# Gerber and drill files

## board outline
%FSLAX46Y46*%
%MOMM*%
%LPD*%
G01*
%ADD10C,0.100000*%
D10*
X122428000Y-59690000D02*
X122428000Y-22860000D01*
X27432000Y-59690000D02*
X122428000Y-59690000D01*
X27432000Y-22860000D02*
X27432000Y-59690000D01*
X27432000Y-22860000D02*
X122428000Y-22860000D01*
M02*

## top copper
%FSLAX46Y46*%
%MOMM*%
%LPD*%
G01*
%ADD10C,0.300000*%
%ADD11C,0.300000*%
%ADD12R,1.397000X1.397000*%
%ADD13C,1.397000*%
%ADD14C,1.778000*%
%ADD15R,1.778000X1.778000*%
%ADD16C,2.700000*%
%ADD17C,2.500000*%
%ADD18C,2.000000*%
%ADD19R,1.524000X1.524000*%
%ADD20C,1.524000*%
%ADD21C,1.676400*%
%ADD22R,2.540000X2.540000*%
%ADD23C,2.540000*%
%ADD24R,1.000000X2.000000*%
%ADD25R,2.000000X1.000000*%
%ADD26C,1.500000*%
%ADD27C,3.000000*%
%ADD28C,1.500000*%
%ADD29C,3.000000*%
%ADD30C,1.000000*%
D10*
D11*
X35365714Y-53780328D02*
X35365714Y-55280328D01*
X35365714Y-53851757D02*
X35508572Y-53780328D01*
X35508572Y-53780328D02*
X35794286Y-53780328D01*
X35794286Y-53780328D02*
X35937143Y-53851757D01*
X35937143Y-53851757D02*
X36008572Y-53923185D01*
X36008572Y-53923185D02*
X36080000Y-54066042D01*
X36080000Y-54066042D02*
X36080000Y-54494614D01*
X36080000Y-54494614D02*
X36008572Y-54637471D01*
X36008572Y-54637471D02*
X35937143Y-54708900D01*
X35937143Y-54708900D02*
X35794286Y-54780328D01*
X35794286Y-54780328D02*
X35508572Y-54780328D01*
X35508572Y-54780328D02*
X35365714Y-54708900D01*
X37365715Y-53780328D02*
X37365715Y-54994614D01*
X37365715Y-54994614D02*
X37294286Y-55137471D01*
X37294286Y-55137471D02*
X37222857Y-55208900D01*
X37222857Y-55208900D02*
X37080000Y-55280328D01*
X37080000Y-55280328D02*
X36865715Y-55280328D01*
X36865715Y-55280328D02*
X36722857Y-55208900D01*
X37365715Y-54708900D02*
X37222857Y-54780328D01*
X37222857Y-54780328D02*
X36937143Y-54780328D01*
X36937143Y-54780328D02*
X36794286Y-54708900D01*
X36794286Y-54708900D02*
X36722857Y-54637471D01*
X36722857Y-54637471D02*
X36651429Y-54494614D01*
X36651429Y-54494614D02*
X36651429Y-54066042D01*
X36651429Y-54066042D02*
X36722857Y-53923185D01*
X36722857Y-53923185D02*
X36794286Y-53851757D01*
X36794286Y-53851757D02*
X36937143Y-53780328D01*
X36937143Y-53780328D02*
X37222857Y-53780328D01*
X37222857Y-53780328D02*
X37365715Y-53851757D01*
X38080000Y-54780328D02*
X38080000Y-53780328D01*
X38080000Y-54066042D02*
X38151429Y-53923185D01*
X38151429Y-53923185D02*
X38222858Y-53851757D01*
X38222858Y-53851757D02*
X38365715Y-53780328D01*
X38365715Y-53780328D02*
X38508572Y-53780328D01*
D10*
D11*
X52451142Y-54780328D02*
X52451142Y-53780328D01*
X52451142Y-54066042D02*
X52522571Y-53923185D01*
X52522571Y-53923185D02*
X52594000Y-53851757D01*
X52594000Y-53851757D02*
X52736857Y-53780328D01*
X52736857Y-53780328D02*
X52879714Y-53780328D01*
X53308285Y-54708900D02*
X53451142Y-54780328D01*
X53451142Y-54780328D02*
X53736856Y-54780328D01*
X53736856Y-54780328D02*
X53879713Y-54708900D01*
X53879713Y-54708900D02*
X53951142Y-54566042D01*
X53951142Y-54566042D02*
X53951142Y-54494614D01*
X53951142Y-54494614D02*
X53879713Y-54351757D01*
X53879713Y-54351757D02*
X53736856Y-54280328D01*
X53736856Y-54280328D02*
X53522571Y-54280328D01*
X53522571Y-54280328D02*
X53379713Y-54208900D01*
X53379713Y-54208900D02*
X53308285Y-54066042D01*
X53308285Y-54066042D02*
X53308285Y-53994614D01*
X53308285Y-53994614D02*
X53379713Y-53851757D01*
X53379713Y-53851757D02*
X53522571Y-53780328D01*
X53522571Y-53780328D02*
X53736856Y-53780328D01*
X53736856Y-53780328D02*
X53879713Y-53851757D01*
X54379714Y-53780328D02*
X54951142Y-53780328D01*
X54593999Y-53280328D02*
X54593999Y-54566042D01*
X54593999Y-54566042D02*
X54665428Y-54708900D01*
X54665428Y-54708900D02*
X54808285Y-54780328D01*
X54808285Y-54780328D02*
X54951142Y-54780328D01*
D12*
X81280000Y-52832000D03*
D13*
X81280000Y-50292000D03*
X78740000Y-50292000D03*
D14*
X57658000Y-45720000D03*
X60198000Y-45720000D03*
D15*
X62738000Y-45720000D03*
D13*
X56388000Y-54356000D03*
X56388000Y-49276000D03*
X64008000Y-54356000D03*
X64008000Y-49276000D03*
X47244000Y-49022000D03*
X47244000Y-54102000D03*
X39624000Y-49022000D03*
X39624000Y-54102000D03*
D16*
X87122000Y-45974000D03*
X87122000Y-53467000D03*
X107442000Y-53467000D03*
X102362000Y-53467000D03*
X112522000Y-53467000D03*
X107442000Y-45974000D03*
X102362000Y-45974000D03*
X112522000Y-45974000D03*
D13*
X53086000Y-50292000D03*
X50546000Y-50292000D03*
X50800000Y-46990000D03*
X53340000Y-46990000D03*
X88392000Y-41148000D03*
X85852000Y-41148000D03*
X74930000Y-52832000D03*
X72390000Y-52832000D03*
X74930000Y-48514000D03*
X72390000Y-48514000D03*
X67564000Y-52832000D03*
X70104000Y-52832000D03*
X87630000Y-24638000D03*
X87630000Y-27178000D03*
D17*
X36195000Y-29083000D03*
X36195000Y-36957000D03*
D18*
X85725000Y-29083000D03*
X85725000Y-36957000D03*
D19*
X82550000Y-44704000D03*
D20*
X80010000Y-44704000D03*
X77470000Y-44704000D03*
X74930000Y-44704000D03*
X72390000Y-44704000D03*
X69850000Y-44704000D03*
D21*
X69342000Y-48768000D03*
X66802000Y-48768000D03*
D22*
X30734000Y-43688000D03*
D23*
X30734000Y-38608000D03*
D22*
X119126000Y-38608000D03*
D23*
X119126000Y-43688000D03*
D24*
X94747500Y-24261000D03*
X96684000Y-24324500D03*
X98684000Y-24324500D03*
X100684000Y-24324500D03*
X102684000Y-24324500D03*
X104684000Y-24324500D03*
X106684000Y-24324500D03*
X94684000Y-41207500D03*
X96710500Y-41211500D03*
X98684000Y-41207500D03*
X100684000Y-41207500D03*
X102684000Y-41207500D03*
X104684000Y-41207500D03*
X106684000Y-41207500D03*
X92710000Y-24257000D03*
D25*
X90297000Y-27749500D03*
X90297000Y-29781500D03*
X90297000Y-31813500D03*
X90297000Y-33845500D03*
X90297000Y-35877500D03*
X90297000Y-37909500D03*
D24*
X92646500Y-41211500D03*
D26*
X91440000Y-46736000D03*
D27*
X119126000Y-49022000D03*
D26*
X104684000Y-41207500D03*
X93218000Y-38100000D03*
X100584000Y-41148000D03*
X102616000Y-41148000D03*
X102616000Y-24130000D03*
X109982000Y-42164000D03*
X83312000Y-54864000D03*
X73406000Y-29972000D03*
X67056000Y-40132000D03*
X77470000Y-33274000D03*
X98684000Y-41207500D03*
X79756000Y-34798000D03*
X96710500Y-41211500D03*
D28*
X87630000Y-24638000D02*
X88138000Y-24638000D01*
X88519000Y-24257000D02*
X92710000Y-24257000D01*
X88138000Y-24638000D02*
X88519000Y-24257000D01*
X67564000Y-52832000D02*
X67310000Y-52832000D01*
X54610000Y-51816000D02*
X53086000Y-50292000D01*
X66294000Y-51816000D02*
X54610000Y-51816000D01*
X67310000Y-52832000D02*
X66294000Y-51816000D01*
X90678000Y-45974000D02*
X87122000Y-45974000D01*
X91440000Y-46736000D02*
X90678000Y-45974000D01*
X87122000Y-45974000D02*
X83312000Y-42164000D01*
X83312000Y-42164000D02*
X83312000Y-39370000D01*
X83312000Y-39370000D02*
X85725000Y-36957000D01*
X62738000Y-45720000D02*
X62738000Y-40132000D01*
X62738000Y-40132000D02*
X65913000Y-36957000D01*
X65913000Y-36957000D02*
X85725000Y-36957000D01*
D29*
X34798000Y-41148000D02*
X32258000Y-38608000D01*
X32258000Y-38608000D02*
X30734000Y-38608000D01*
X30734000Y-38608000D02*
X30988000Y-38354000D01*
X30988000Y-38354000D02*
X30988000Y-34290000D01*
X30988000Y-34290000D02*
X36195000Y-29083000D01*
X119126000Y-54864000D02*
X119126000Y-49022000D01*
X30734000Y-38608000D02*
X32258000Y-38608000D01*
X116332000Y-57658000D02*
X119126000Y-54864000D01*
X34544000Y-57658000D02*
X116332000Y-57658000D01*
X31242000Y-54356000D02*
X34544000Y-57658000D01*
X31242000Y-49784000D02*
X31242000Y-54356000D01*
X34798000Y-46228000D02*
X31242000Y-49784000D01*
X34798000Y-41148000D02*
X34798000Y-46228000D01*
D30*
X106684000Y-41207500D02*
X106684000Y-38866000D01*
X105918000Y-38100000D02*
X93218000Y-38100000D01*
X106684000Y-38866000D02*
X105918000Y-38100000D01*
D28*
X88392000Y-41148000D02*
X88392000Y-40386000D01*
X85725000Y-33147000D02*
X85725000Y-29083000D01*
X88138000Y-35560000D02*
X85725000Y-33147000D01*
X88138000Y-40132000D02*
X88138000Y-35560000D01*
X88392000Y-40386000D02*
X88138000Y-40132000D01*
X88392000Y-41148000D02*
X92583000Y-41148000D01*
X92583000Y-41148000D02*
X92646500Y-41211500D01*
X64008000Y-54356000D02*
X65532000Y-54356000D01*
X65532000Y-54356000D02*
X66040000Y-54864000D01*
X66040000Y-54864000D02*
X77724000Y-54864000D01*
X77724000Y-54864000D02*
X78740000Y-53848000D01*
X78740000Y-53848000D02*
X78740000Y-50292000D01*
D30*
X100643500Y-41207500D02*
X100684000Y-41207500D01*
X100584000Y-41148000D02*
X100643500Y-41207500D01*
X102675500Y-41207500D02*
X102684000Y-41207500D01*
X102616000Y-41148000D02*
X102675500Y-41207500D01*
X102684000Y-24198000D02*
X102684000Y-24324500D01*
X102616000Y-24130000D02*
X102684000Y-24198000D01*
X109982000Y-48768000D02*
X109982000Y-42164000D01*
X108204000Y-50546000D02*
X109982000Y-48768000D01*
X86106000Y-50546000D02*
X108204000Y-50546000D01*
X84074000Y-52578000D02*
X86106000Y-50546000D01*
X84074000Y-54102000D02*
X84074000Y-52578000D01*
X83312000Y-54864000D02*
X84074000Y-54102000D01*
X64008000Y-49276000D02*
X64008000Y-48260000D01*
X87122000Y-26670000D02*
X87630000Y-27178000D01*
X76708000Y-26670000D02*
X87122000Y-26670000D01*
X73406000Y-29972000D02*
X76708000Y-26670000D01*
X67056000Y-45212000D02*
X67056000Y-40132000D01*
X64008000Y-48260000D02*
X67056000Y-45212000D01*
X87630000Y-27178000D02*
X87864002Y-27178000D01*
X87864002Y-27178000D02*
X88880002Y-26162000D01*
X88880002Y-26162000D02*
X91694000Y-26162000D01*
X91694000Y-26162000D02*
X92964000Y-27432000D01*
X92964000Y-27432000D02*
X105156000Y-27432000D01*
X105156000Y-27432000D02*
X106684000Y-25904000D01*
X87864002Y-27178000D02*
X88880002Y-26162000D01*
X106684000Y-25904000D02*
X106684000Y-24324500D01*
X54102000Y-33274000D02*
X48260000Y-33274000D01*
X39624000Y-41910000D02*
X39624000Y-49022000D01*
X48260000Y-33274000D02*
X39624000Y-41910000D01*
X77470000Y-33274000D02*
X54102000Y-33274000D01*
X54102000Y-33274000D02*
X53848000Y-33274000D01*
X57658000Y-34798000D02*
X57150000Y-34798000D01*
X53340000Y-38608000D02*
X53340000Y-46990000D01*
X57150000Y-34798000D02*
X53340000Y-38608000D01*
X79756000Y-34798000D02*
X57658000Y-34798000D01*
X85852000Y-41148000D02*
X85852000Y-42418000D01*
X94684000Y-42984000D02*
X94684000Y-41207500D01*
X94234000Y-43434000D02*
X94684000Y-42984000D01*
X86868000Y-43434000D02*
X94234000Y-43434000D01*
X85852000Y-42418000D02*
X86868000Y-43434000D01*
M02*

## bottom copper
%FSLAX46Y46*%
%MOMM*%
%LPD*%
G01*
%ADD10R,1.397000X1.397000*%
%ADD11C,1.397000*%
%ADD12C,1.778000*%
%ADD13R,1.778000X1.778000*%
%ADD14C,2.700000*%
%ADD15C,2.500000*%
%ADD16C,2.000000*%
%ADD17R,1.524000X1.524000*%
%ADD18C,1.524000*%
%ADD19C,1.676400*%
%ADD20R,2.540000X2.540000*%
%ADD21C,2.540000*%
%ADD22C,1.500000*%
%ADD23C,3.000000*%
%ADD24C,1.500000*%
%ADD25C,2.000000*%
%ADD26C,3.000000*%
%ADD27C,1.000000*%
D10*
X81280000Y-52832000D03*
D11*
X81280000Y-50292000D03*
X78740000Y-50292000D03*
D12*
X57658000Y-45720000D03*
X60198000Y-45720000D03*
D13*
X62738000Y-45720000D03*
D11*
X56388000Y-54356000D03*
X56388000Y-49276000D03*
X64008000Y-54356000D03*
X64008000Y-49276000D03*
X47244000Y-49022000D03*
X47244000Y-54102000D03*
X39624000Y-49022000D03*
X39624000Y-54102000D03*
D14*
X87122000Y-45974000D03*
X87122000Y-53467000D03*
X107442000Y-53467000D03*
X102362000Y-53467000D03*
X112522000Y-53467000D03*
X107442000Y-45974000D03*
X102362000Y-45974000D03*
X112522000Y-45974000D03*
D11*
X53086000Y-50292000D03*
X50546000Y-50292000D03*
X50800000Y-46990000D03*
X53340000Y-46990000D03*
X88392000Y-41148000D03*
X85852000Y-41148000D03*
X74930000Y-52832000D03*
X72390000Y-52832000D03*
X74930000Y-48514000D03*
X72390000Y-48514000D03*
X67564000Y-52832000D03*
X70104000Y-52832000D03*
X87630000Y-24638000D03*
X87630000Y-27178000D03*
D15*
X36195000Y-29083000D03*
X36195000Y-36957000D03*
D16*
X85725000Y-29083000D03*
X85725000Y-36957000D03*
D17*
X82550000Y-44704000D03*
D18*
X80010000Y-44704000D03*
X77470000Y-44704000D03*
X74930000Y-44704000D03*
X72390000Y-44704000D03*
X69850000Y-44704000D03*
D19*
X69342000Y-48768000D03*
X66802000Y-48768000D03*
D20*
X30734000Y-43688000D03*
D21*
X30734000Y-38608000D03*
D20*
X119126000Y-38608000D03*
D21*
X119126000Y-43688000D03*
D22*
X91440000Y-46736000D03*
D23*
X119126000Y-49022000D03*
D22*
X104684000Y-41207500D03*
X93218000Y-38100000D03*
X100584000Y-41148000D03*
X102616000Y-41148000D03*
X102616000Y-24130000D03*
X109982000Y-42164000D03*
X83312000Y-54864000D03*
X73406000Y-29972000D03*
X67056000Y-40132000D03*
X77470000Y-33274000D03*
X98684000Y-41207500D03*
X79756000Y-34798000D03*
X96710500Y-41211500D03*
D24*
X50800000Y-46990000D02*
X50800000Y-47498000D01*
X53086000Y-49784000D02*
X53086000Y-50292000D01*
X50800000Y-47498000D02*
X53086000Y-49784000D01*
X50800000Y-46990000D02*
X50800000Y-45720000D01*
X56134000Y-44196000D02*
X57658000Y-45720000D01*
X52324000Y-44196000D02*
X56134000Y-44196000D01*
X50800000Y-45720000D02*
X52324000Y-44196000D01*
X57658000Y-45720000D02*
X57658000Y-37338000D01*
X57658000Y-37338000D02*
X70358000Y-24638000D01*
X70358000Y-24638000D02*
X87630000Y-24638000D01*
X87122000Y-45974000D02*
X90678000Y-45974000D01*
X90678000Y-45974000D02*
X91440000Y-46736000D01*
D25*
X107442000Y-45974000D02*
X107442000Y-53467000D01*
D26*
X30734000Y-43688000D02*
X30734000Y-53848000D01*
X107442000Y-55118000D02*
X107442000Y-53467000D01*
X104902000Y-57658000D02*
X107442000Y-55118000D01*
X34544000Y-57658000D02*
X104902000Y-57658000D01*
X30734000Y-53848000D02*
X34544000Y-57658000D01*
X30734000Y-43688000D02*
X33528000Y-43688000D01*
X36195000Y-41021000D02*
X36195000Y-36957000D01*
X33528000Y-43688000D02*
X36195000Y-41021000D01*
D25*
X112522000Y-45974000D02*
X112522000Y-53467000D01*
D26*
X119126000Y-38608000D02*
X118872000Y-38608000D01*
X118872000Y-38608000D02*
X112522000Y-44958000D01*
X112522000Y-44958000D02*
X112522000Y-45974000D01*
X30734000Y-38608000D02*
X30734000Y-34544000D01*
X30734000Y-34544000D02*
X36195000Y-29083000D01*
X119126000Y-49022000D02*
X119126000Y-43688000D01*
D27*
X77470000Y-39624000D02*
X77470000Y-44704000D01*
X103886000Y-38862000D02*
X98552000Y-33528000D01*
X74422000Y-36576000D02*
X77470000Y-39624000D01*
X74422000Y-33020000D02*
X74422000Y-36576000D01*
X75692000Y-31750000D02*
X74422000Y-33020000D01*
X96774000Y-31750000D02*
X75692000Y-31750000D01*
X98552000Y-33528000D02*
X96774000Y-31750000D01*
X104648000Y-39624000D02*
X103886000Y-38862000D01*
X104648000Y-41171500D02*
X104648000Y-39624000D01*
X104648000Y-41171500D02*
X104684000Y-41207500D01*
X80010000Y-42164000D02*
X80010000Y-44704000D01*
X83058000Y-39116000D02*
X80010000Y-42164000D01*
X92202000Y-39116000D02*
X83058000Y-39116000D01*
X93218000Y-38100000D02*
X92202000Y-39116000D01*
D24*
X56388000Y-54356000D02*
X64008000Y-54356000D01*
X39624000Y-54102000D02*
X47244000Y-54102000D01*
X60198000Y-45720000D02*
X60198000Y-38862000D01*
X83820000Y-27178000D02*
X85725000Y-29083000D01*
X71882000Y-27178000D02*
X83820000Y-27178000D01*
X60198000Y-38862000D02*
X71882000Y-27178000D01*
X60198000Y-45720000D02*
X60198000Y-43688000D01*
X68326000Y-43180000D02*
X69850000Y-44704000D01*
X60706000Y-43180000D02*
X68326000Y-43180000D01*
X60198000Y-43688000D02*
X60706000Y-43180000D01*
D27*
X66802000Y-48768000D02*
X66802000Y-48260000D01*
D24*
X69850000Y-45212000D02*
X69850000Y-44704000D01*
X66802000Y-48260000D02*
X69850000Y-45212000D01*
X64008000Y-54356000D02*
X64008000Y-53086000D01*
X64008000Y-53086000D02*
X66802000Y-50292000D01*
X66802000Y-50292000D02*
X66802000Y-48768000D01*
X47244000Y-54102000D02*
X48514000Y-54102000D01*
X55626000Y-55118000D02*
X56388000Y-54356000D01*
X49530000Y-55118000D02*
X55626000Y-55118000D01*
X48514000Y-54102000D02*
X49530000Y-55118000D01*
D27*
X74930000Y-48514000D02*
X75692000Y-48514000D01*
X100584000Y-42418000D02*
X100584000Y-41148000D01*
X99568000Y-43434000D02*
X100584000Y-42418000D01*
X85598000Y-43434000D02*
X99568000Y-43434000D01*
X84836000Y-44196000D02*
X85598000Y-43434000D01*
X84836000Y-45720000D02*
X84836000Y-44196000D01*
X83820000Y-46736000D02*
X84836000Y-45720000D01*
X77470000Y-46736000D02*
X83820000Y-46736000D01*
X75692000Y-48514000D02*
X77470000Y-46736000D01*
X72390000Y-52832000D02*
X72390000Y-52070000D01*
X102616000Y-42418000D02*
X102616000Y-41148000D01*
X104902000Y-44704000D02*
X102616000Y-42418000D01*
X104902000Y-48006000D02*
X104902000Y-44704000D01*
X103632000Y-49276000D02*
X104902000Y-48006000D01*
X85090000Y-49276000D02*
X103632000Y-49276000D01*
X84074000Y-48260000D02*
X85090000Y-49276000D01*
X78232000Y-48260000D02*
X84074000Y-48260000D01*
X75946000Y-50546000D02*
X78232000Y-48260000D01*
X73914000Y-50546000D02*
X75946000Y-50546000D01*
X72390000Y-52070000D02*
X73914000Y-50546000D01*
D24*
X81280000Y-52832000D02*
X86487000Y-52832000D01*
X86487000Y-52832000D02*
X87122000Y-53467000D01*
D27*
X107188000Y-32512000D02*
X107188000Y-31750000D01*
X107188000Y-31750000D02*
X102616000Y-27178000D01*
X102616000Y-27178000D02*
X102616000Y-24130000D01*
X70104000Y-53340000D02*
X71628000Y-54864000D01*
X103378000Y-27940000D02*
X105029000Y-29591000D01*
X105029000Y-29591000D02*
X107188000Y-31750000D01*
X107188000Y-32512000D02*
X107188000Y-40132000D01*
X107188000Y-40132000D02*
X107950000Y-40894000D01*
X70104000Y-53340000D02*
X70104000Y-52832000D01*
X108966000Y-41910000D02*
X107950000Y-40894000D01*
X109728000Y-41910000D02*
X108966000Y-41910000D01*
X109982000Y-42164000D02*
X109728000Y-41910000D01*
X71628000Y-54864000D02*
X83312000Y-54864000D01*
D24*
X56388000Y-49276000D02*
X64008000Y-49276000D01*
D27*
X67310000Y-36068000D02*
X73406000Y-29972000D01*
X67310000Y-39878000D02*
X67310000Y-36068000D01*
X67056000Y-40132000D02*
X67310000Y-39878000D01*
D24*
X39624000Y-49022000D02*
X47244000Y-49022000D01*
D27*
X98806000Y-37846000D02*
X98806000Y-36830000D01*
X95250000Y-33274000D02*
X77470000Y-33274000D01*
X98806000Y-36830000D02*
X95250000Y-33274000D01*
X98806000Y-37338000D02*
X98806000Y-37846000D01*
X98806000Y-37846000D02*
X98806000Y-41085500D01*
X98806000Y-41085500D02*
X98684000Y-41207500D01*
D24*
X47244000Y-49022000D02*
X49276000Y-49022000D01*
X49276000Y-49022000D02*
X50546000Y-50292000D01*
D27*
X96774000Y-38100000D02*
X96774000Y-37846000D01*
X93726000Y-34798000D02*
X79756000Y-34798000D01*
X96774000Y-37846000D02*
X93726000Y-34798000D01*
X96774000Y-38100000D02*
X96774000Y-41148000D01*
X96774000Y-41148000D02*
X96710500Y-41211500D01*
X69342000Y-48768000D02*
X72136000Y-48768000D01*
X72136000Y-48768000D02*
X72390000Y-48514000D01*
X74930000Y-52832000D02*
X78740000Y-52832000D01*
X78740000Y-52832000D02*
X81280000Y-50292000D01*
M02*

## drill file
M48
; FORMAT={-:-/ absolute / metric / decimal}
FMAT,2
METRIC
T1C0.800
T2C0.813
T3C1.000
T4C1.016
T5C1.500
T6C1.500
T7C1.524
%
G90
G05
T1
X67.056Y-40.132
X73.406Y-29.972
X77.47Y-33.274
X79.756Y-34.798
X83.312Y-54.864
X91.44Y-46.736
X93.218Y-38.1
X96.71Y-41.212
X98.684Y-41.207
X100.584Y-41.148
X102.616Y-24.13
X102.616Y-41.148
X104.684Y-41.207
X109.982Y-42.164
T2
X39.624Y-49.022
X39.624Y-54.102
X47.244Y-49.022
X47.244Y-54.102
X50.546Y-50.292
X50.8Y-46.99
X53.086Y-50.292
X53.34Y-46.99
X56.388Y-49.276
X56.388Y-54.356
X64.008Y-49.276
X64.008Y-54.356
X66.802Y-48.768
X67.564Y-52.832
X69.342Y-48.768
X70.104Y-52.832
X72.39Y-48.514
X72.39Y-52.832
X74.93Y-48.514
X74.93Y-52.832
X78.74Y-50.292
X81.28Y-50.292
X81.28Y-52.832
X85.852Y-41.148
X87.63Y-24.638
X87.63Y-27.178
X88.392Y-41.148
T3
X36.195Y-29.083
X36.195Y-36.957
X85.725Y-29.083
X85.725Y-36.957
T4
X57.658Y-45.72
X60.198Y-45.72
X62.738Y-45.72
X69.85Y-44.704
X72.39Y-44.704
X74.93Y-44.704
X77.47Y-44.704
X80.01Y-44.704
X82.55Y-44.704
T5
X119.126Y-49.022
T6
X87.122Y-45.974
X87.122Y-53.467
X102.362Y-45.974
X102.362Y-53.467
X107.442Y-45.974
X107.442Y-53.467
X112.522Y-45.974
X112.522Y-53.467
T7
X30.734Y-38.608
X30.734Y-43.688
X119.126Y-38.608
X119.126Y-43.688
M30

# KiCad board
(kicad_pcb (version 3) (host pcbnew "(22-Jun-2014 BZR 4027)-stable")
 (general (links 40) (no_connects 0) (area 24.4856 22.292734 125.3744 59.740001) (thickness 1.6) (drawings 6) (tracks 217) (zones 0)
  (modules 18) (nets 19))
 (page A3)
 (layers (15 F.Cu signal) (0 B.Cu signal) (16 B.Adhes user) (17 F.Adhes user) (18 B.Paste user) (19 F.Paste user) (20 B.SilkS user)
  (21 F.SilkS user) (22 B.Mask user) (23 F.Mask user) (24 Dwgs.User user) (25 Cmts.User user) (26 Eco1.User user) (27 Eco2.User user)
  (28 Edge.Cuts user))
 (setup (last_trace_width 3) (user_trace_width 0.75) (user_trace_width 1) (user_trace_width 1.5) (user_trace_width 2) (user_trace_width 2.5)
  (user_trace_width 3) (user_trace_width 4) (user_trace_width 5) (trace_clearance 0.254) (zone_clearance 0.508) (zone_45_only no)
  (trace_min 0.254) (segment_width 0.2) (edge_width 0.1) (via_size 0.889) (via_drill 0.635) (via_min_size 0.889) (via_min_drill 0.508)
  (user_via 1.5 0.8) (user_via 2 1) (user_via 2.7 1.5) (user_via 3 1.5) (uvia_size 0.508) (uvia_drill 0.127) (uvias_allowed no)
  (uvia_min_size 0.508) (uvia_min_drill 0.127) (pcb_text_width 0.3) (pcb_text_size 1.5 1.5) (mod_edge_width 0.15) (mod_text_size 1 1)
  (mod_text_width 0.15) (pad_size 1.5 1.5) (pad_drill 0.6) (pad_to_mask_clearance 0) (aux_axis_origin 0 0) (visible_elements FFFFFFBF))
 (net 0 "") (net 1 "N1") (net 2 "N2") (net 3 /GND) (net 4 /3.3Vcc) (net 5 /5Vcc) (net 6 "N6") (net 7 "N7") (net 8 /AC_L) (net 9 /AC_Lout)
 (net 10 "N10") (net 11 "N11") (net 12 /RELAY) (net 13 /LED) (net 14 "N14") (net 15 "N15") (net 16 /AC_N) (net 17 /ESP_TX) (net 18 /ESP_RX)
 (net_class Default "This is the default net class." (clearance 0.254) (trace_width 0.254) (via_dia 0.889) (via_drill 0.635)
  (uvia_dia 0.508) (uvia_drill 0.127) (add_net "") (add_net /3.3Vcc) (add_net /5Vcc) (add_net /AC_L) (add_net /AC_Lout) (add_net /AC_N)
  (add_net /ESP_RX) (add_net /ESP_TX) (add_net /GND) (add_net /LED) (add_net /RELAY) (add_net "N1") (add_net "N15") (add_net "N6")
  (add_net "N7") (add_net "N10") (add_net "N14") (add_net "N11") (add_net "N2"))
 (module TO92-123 (layer F.Cu) (at 80.01 51.562 270)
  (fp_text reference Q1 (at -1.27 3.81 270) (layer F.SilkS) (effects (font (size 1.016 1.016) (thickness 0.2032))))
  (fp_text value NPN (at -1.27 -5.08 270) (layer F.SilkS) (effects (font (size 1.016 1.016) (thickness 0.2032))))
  (pad 3 thru_hole rect (at 1.27 -1.27 270) (size 1.397 1.397) (drill 0.8128) (layers *.Cu *.Mask F.SilkS) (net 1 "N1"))
  (pad 2 thru_hole circle (at -1.27 -1.27 270) (size 1.397 1.397) (drill 0.8128) (layers *.Cu *.Mask F.SilkS) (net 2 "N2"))
  (pad 1 thru_hole circle (at -1.27 1.27 270) (size 1.397 1.397) (drill 0.8128) (layers *.Cu *.Mask F.SilkS) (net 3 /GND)))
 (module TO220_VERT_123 (layer F.Cu) (at 60.198 45.72 90)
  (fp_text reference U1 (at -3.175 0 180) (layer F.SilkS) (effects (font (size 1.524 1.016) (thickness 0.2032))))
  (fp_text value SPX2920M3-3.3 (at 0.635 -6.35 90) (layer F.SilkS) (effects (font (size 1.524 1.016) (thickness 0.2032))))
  (pad 3 thru_hole circle (at 0 -2.54 90) (size 1.778 1.778) (drill 1.016) (layers *.Cu *.Mask F.SilkS) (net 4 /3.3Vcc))
  (pad 2 thru_hole circle (at 0 0 90) (size 1.778 1.778) (drill 1.016) (layers *.Cu *.Mask F.SilkS) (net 3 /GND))
  (pad 1 thru_hole rect (at 0 2.54 90) (size 1.778 1.778) (drill 1.016) (layers *.Cu *.Mask F.SilkS) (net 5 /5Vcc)))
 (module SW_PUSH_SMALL (layer F.Cu) (at 60.198 51.816 180)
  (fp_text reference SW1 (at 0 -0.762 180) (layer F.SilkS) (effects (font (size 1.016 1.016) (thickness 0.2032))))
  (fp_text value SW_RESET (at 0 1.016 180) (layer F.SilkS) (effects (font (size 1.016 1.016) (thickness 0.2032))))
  (pad 1 thru_hole circle (at 3.81 -2.54 180) (size 1.397 1.397) (drill 0.8128) (layers *.Cu *.Mask F.SilkS) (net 3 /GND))
  (pad 2 thru_hole circle (at 3.81 2.54 180) (size 1.397 1.397) (drill 0.8128) (layers *.Cu *.Mask F.SilkS) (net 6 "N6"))
  (pad 1 thru_hole circle (at -3.81 -2.54 180) (size 1.397 1.397) (drill 0.8128) (layers *.Cu *.Mask F.SilkS) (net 3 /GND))
  (pad 2 thru_hole circle (at -3.81 2.54 180) (size 1.397 1.397) (drill 0.8128) (layers *.Cu *.Mask F.SilkS) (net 6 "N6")))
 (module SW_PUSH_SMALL (layer F.Cu) (at 43.434 51.562)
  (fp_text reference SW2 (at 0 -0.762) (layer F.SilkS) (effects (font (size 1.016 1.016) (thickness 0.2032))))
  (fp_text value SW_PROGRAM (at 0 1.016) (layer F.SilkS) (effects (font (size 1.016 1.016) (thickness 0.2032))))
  (pad 1 thru_hole circle (at 3.81 -2.54) (size 1.397 1.397) (drill 0.8128) (layers *.Cu *.Mask F.SilkS) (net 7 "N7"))
  (pad 2 thru_hole circle (at 3.81 2.54) (size 1.397 1.397) (drill 0.8128) (layers *.Cu *.Mask F.SilkS) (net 3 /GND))
  (pad 1 thru_hole circle (at -3.81 -2.54) (size 1.397 1.397) (drill 0.8128) (layers *.Cu *.Mask F.SilkS) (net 7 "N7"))
  (pad 2 thru_hole circle (at -3.81 2.54) (size 1.397 1.397) (drill 0.8128) (layers *.Cu *.Mask F.SilkS) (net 3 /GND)))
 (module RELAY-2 (layer F.Cu) (at 88.646 44.196)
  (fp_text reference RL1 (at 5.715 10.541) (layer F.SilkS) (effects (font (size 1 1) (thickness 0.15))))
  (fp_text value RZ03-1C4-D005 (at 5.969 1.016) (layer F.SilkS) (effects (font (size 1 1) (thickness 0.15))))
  (pad 1 thru_hole circle (at -1.524 1.778) (size 2.7 2.7) (drill 1.5) (layers *.Cu *.Mask F.SilkS) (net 5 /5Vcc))
  (pad 2 thru_hole circle (at -1.524 9.271) (size 2.7 2.7) (drill 1.5) (layers *.Cu *.Mask F.SilkS) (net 1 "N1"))
  (pad 11 thru_hole circle (at 18.796 9.271) (size 2.7 2.7) (drill 1.5) (layers *.Cu *.Mask F.SilkS) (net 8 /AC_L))
  (pad 12 thru_hole circle (at 13.716 9.271) (size 2.7 2.7) (drill 1.5) (layers *.Cu *.Mask F.SilkS))
  (pad 14 thru_hole circle (at 23.876 9.271) (size 2.7 2.7) (drill 1.5) (layers *.Cu *.Mask F.SilkS) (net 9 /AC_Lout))
  (pad 11 thru_hole circle (at 18.796 1.778) (size 2.7 2.7) (drill 1.5) (layers *.Cu *.Mask F.SilkS) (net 8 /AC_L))
  (pad 12 thru_hole circle (at 13.716 1.778) (size 2.7 2.7) (drill 1.5) (layers *.Cu *.Mask F.SilkS))
  (pad 14 thru_hole circle (at 23.876 1.778) (size 2.7 2.7) (drill 1.5) (layers *.Cu *.Mask F.SilkS) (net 9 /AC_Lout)))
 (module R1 (layer F.Cu) (at 51.816 50.292 180) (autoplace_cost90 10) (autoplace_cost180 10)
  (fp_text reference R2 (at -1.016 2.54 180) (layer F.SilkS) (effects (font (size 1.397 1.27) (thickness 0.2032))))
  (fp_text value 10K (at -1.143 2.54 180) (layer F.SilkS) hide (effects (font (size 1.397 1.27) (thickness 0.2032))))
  (pad 1 thru_hole circle (at -1.27 0 180) (size 1.397 1.397) (drill 0.8128) (layers *.Cu *.Mask F.SilkS) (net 4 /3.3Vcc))
  (pad 2 thru_hole circle (at 1.27 0 180) (size 1.397 1.397) (drill 0.8128) (layers *.Cu *.Mask F.SilkS) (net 7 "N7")))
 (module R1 (layer F.Cu) (at 52.07 46.99) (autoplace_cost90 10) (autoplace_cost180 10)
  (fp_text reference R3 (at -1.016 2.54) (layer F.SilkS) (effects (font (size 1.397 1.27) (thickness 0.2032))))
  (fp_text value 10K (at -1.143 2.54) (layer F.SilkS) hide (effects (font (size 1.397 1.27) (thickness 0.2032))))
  (pad 1 thru_hole circle (at -1.27 0) (size 1.397 1.397) (drill 0.8128) (layers *.Cu *.Mask F.SilkS) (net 4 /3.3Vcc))
  (pad 2 thru_hole circle (at 1.27 0) (size 1.397 1.397) (drill 0.8128) (layers *.Cu *.Mask F.SilkS) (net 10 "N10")))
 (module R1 (layer F.Cu) (at 87.122 41.148 180) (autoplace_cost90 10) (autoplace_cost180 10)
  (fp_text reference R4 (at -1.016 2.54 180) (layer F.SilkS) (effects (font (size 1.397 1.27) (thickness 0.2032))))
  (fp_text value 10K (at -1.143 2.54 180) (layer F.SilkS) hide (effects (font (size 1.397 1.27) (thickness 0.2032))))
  (pad 1 thru_hole circle (at -1.27 0 180) (size 1.397 1.397) (drill 0.8128) (layers *.Cu *.Mask F.SilkS) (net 3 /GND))
  (pad 2 thru_hole circle (at 1.27 0 180) (size 1.397 1.397) (drill 0.8128) (layers *.Cu *.Mask F.SilkS) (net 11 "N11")))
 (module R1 (layer F.Cu) (at 73.66 52.832 180) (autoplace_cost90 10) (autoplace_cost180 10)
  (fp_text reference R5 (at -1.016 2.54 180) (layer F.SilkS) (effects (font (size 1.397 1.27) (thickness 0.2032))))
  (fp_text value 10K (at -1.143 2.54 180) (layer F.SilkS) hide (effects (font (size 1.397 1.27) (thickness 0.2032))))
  (pad 1 thru_hole circle (at -1.27 0 180) (size 1.397 1.397) (drill 0.8128) (layers *.Cu *.Mask F.SilkS) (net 2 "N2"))
  (pad 2 thru_hole circle (at 1.27 0 180) (size 1.397 1.397) (drill 0.8128) (layers *.Cu *.Mask F.SilkS) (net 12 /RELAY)))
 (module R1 (layer F.Cu) (at 73.66 48.514 180) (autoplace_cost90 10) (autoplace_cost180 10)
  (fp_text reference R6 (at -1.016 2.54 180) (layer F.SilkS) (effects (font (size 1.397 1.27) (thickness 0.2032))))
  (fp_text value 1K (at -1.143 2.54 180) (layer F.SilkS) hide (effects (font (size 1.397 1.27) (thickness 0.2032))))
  (pad 1 thru_hole circle (at -1.27 0 180) (size 1.397 1.397) (drill 0.8128) (layers *.Cu *.Mask F.SilkS) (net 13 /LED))
  (pad 2 thru_hole circle (at 1.27 0 180) (size 1.397 1.397) (drill 0.8128) (layers *.Cu *.Mask F.SilkS) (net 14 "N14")))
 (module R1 (layer F.Cu) (at 68.834 52.832) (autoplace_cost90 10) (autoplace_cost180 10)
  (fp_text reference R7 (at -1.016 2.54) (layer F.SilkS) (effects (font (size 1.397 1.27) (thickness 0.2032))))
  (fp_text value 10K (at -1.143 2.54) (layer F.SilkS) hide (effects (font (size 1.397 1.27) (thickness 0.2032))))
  (pad 1 thru_hole circle (at -1.27 0) (size 1.397 1.397) (drill 0.8128) (layers *.Cu *.Mask F.SilkS) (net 4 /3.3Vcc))
  (pad 2 thru_hole circle (at 1.27 0) (size 1.397 1.397) (drill 0.8128) (layers *.Cu *.Mask F.SilkS) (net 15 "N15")))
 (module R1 (layer F.Cu) (at 87.63 25.908 270) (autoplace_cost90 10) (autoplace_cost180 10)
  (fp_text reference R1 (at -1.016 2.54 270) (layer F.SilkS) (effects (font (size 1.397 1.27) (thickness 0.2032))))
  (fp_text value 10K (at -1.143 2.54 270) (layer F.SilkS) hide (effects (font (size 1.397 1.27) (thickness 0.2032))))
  (pad 1 thru_hole circle (at -1.27 0 270) (size 1.397 1.397) (drill 0.8128) (layers *.Cu *.Mask F.SilkS) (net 4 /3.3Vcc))
  (pad 2 thru_hole circle (at 1.27 0 270) (size 1.397 1.397) (drill 0.8128) (layers *.Cu *.Mask F.SilkS) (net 6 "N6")))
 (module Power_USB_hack (layer F.Cu) (at 60.96 33.02)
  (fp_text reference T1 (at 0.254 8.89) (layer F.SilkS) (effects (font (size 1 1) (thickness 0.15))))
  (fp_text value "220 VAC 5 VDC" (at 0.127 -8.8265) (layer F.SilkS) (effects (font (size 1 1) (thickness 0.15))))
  (pad 1 thru_hole circle (at -24.765 -3.937) (size 2.5 2.5) (drill 1) (layers *.Cu *.Mask F.SilkS) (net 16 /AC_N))
  (pad 2 thru_hole circle (at -24.765 3.937) (size 2.5 2.5) (drill 1) (layers *.Cu *.Mask F.SilkS) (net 8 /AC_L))
  (pad 4 thru_hole circle (at 24.765 -3.937) (size 2 2) (drill 1) (layers *.Cu *.Mask F.SilkS) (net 3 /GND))
  (pad 3 thru_hole circle (at 24.765 3.937) (size 2 2) (drill 1) (layers *.Cu *.Mask F.SilkS) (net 5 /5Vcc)))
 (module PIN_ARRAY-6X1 (layer F.Cu) (at 76.2 44.704 180)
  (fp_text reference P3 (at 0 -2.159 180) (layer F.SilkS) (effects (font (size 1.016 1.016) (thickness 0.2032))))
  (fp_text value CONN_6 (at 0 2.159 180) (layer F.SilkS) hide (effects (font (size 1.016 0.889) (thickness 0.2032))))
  (pad 1 thru_hole rect (at -6.35 0 180) (size 1.524 1.524) (drill 1.016) (layers *.Cu *.Mask F.SilkS))
  (pad 2 thru_hole circle (at -3.81 0 180) (size 1.524 1.524) (drill 1.016) (layers *.Cu *.Mask F.SilkS) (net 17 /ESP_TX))
  (pad 3 thru_hole circle (at -1.27 0 180) (size 1.524 1.524) (drill 1.016) (layers *.Cu *.Mask F.SilkS) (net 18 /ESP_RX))
  (pad 4 thru_hole circle (at 1.27 0 180) (size 1.524 1.524) (drill 1.016) (layers *.Cu *.Mask F.SilkS))
  (pad 5 thru_hole circle (at 3.81 0 180) (size 1.524 1.524) (drill 1.016) (layers *.Cu *.Mask F.SilkS))
  (pad 6 thru_hole circle (at 6.35 0 180) (size 1.524 1.524) (drill 1.016) (layers *.Cu *.Mask F.SilkS) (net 3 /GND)))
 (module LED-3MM (layer F.Cu) (at 68.072 48.768 180)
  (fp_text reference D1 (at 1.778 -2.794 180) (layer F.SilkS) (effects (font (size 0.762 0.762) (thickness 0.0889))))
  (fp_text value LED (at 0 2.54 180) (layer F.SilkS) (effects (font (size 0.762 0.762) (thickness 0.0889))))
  (pad 1 thru_hole circle (at -1.27 0 180) (size 1.6764 1.6764) (drill 0.8128) (layers *.Cu *.Mask F.SilkS) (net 14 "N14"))
  (pad 2 thru_hole circle (at 1.27 0 180) (size 1.6764 1.6764) (drill 0.8128) (layers *.Cu *.Mask F.SilkS) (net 3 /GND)))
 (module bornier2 (layer F.Cu) (at 30.734 41.148 90)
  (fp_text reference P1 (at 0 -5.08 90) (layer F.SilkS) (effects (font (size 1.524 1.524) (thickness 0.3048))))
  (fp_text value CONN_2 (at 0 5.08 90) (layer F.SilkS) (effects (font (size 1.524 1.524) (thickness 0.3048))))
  (pad 1 thru_hole rect (at -2.54 0 90) (size 2.54 2.54) (drill 1.524) (layers *.Cu *.Mask F.SilkS) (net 8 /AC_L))
  (pad 2 thru_hole circle (at 2.54 0 90) (size 2.54 2.54) (drill 1.524) (layers *.Cu *.Mask F.SilkS) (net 16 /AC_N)))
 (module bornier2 (layer F.Cu) (at 119.126 41.148 270)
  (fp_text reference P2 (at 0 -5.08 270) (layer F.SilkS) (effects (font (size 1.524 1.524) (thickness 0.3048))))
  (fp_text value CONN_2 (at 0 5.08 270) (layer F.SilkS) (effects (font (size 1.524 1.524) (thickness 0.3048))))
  (pad 1 thru_hole rect (at -2.54 0 270) (size 2.54 2.54) (drill 1.524) (layers *.Cu *.Mask F.SilkS) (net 9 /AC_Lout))
  (pad 2 thru_hole circle (at 2.54 0 270) (size 2.54 2.54) (drill 1.524) (layers *.Cu *.Mask F.SilkS) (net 16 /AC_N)))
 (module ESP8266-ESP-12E (layer F.Cu) (at 102.87 32.766 270)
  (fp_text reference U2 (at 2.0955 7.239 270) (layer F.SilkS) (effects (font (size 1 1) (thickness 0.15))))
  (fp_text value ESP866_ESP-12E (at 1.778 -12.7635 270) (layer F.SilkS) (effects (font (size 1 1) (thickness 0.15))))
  (pad 7 smd rect (at -8.505 8.1225 270) (size 2 1) (layers F.Cu F.Paste F.Mask))
  (pad 6 smd rect (at -8.4415 6.186 270) (size 2 1) (layers F.Cu F.Paste F.Mask))
  (pad 5 smd rect (at -8.4415 4.186 270) (size 2 1) (layers F.Cu F.Paste F.Mask))
  (pad 4 smd rect (at -8.4415 2.186 270) (size 2 1) (layers F.Cu F.Paste F.Mask))
  (pad 3 smd rect (at -8.4415 0.186 270) (size 2 1) (layers F.Cu F.Paste F.Mask) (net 15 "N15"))
  (pad 2 smd rect (at -8.4415 -1.814 270) (size 2 1) (layers F.Cu F.Paste F.Mask))
  (pad 1 smd rect (at -8.4415 -3.814 270) (size 2 1) (layers F.Cu F.Paste F.Mask) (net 6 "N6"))
  (pad 16 smd rect (at 8.4415 8.186 270) (size 2 1) (layers F.Cu F.Paste F.Mask) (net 11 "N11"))
  (pad 17 smd rect (at 8.4455 6.1595 270) (size 2 1) (layers F.Cu F.Paste F.Mask) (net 10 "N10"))
  (pad 18 smd rect (at 8.4415 4.186 270) (size 2 1) (layers F.Cu F.Paste F.Mask) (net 7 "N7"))
  (pad 19 smd rect (at 8.4415 2.186 270) (size 2 1) (layers F.Cu F.Paste F.Mask) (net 13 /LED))
  (pad 20 smd rect (at 8.4415 0.186 270) (size 2 1) (layers F.Cu F.Paste F.Mask) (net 12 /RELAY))
  (pad 21 smd rect (at 8.4415 -1.814 270) (size 2 1) (layers F.Cu F.Paste F.Mask) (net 18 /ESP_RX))
  (pad 22 smd rect (at 8.4415 -3.814 270) (size 2 1) (layers F.Cu F.Paste F.Mask) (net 17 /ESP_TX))
  (pad 8 smd rect (at -8.509 10.16 270) (size 2 1) (layers F.Cu F.Paste F.Mask) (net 4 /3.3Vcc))
  (pad 9 smd rect (at -5.0165 12.573) (size 2 1) (layers F.Cu F.Paste F.Mask))
  (pad 10 smd rect (at -2.9845 12.573) (size 2 1) (layers F.Cu F.Paste F.Mask))
  (pad 11 smd rect (at -0.9525 12.573) (size 2 1) (layers F.Cu F.Paste F.Mask))
  (pad 12 smd rect (at 1.0795 12.573) (size 2 1) (layers F.Cu F.Paste F.Mask))
  (pad 13 smd rect (at 3.1115 12.573) (size 2 1) (layers F.Cu F.Paste F.Mask))
  (pad 14 smd rect (at 5.1435 12.573) (size 2 1) (layers F.Cu F.Paste F.Mask))
  (pad 15 smd rect (at 8.4455 10.2235 270) (size 2 1) (layers F.Cu F.Paste F.Mask) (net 3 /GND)))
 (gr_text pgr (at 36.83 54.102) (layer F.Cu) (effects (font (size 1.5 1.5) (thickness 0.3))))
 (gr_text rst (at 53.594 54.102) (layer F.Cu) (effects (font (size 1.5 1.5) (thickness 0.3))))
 (gr_line (start 122.428 59.69) (end 122.428 22.86) (angle 90) (layer Edge.Cuts) (width 0.1))
 (gr_line (start 27.432 59.69) (end 122.428 59.69) (angle 90) (layer Edge.Cuts) (width 0.1))
 (gr_line (start 27.432 22.86) (end 27.432 59.69) (angle 90) (layer Edge.Cuts) (width 0.1))
 (gr_line (start 27.432 22.86) (end 122.428 22.86) (angle 90) (layer Edge.Cuts) (width 0.1))
 (segment (start 87.63 24.638) (end 88.138 24.638) (width 1.5) (layer F.Cu) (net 4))
 (segment (start 88.519 24.257) (end 92.71 24.257) (width 1.5) (layer F.Cu) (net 4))
 (segment (start 88.138 24.638) (end 88.519 24.257) (width 1.5) (layer F.Cu) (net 4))
 (segment (start 67.564 52.832) (end 67.31 52.832) (width 1.5) (layer F.Cu) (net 4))
 (segment (start 54.61 51.816) (end 53.086 50.292) (width 1.5) (layer F.Cu) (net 4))
 (segment (start 66.294 51.816) (end 54.61 51.816) (width 1.5) (layer F.Cu) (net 4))
 (segment (start 67.31 52.832) (end 66.294 51.816) (width 1.5) (layer F.Cu) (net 4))
 (segment (start 50.8 46.99) (end 50.8 47.498) (width 1.5) (layer B.Cu) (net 4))
 (segment (start 53.086 49.784) (end 53.086 50.292) (width 1.5) (layer B.Cu) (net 4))
 (segment (start 50.8 47.498) (end 53.086 49.784) (width 1.5) (layer B.Cu) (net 4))
 (segment (start 50.8 46.99) (end 50.8 45.72) (width 1.5) (layer B.Cu) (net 4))
 (segment (start 56.134 44.196) (end 57.658 45.72) (width 1.5) (layer B.Cu) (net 4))
 (segment (start 52.324 44.196) (end 56.134 44.196) (width 1.5) (layer B.Cu) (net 4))
 (segment (start 50.8 45.72) (end 52.324 44.196) (width 1.5) (layer B.Cu) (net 4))
 (segment (start 57.658 45.72) (end 57.658 37.338) (width 1.5) (layer B.Cu) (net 4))
 (segment (start 57.658 37.338) (end 70.358 24.638) (width 1.5) (layer B.Cu) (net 4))
 (segment (start 70.358 24.638) (end 87.63 24.638) (width 1.5) (layer B.Cu) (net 4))
 (segment (start 87.122 45.974) (end 90.678 45.974) (width 1.5) (layer B.Cu) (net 5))
 (segment (start 90.678 45.974) (end 87.122 45.974) (width 1.5) (layer F.Cu) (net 5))
 (segment (start 91.44 46.736) (end 90.678 45.974) (width 1.5) (layer F.Cu) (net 5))
 (via (at 91.44 46.736) (size 1.5) (drill 0.8) (layers F.Cu B.Cu) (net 5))
 (segment (start 90.678 45.974) (end 91.44 46.736) (width 1.5) (layer B.Cu) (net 5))
 (segment (start 87.122 45.974) (end 83.312 42.164) (width 1.5) (layer F.Cu) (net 5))
 (segment (start 83.312 42.164) (end 83.312 39.37) (width 1.5) (layer F.Cu) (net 5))
 (segment (start 83.312 39.37) (end 85.725 36.957) (width 1.5) (layer F.Cu) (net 5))
 (segment (start 62.738 45.72) (end 62.738 40.132) (width 1.5) (layer F.Cu) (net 5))
 (segment (start 62.738 40.132) (end 65.913 36.957) (width 1.5) (layer F.Cu) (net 5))
 (segment (start 65.913 36.957) (end 85.725 36.957) (width 1.5) (layer F.Cu) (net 5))
 (segment (start 107.442 45.974) (end 107.442 53.467) (width 2) (layer B.Cu) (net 8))
 (segment (start 30.734 43.688) (end 30.734 53.848) (width 3) (layer B.Cu) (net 8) (status 10))
 (segment (start 107.442 55.118) (end 107.442 53.467) (width 3) (layer B.Cu) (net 8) (status 20))
 (segment (start 104.902 57.658) (end 107.442 55.118) (width 3) (layer B.Cu) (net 8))
 (segment (start 34.544 57.658) (end 104.902 57.658) (width 3) (layer B.Cu) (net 8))
 (segment (start 30.734 53.848) (end 34.544 57.658) (width 3) (layer B.Cu) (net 8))
 (segment (start 30.734 43.688) (end 33.528 43.688) (width 3) (layer B.Cu) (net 8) (status 10))
 (segment (start 36.195 41.021) (end 36.195 36.957) (width 3) (layer B.Cu) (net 8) (status 20))
 (segment (start 33.528 43.688) (end 36.195 41.021) (width 3) (layer B.Cu) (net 8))
 (segment (start 112.522 45.974) (end 112.522 53.467) (width 2) (layer B.Cu) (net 9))
 (segment (start 119.126 38.608) (end 118.872 38.608) (width 3) (layer B.Cu) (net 9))
 (segment (start 118.872 38.608) (end 112.522 44.958) (width 3) (layer B.Cu) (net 9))
 (segment (start 112.522 44.958) (end 112.522 45.974) (width 3) (layer B.Cu) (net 9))
 (segment (start 34.798 41.148) (end 32.258 38.608) (width 3) (layer F.Cu) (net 16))
 (segment (start 32.258 38.608) (end 30.734 38.608) (width 3) (layer F.Cu) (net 16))
 (segment (start 30.734 38.608) (end 30.988 38.354) (width 3) (layer F.Cu) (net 16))
 (segment (start 30.988 38.354) (end 30.988 34.29) (width 3) (layer F.Cu) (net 16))
 (segment (start 30.988 34.29) (end 36.195 29.083) (width 3) (layer F.Cu) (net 16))
 (segment (start 30.734 38.608) (end 30.734 34.544) (width 3) (layer B.Cu) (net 16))
 (segment (start 30.734 34.544) (end 36.195 29.083) (width 3) (layer B.Cu) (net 16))
 (segment (start 119.126 54.864) (end 119.126 49.022) (width 3) (layer F.Cu) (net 16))
 (segment (start 119.126 49.022) (end 119.126 43.688) (width 3) (layer B.Cu) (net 16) (status 20))
 (via (at 119.126 49.022) (size 3) (drill 1.5) (layers F.Cu B.Cu) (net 16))
 (segment (start 30.734 38.608) (end 32.258 38.608) (width 3) (layer F.Cu) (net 16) (status 10))
 (segment (start 116.332 57.658) (end 119.126 54.864) (width 3) (layer F.Cu) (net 16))
 (segment (start 34.544 57.658) (end 116.332 57.658) (width 3) (layer F.Cu) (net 16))
 (segment (start 31.242 54.356) (end 34.544 57.658) (width 3) (layer F.Cu) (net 16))
 (segment (start 31.242 49.784) (end 31.242 54.356) (width 3) (layer F.Cu) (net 16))
 (segment (start 34.798 46.228) (end 31.242 49.784) (width 3) (layer F.Cu) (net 16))
 (segment (start 34.798 41.148) (end 34.798 46.228) (width 3) (layer F.Cu) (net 16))
 (segment (start 77.47 39.624) (end 77.47 44.704) (width 1) (layer B.Cu) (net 18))
 (segment (start 103.886 38.862) (end 98.552 33.528) (width 1) (layer B.Cu) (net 18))
 (segment (start 74.422 36.576) (end 77.47 39.624) (width 1) (layer B.Cu) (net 18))
 (segment (start 74.422 33.02) (end 74.422 36.576) (width 1) (layer B.Cu) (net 18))
 (segment (start 75.692 31.75) (end 74.422 33.02) (width 1) (layer B.Cu) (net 18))
 (segment (start 96.774 31.75) (end 75.692 31.75) (width 1) (layer B.Cu) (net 18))
 (segment (start 98.552 33.528) (end 96.774 31.75) (width 1) (layer B.Cu) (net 18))
 (via (at 104.684 41.2075) (size 1.5) (drill 0.8) (layers F.Cu B.Cu) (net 18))
 (segment (start 104.648 39.624) (end 103.886 38.862) (width 1) (layer B.Cu) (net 18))
 (segment (start 104.648 41.1715) (end 104.648 39.624) (width 1) (layer B.Cu) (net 18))
 (segment (start 104.648 41.1715) (end 104.684 41.2075) (width 1) (layer B.Cu) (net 18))
 (segment (start 106.684 41.2075) (end 106.684 38.866) (width 1) (layer F.Cu) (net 17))
 (segment (start 80.01 42.164) (end 80.01 44.704) (width 1) (layer B.Cu) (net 17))
 (segment (start 83.058 39.116) (end 80.01 42.164) (width 1) (layer B.Cu) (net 17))
 (segment (start 92.202 39.116) (end 83.058 39.116) (width 1) (layer B.Cu) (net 17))
 (segment (start 93.218 38.1) (end 92.202 39.116) (width 1) (layer B.Cu) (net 17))
 (via (at 93.218 38.1) (size 1.5) (drill 0.8) (layers F.Cu B.Cu) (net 17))
 (segment (start 105.918 38.1) (end 93.218 38.1) (width 1) (layer F.Cu) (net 17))
 (segment (start 106.684 38.866) (end 105.918 38.1) (width 1) (layer F.Cu) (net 17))
 (segment (start 56.388 54.356) (end 64.008 54.356) (width 1.5) (layer B.Cu) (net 3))
 (segment (start 39.624 54.102) (end 47.244 54.102) (width 1.5) (layer B.Cu) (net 3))
 (segment (start 88.392 41.148) (end 88.392 40.386) (width 1.5) (layer F.Cu) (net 3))
 (segment (start 85.725 33.147) (end 85.725 29.083) (width 1.5) (layer F.Cu) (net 3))
 (segment (start 88.138 35.56) (end 85.725 33.147) (width 1.5) (layer F.Cu) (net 3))
 (segment (start 88.138 40.132) (end 88.138 35.56) (width 1.5) (layer F.Cu) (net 3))
 (segment (start 88.392 40.386) (end 88.138 40.132) (width 1.5) (layer F.Cu) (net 3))
 (segment (start 60.198 45.72) (end 60.198 38.862) (width 1.5) (layer B.Cu) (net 3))
 (segment (start 83.82 27.178) (end 85.725 29.083) (width 1.5) (layer B.Cu) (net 3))
 (segment (start 71.882 27.178) (end 83.82 27.178) (width 1.5) (layer B.Cu) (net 3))
 (segment (start 60.198 38.862) (end 71.882 27.178) (width 1.5) (layer B.Cu) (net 3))
 (segment (start 88.392 41.148) (end 92.583 41.148) (width 1.5) (layer F.Cu) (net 3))
 (segment (start 92.583 41.148) (end 92.6465 41.2115) (width 1.5) (layer F.Cu) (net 3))
 (segment (start 64.008 54.356) (end 65.532 54.356) (width 1.5) (layer F.Cu) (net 3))
 (segment (start 65.532 54.356) (end 66.04 54.864) (width 1.5) (layer F.Cu) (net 3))
 (segment (start 66.04 54.864) (end 77.724 54.864) (width 1.5) (layer F.Cu) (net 3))
 (segment (start 77.724 54.864) (end 78.74 53.848) (width 1.5) (layer F.Cu) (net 3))
 (segment (start 78.74 53.848) (end 78.74 50.292) (width 1.5) (layer F.Cu) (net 3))
 (segment (start 60.198 45.72) (end 60.198 43.688) (width 1.5) (layer B.Cu) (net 3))
 (segment (start 68.326 43.18) (end 69.85 44.704) (width 1.5) (layer B.Cu) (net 3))
 (segment (start 60.706 43.18) (end 68.326 43.18) (width 1.5) (layer B.Cu) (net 3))
 (segment (start 60.198 43.688) (end 60.706 43.18) (width 1.5) (layer B.Cu) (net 3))
 (segment (start 66.802 48.768) (end 66.802 48.26) (width 1) (layer B.Cu) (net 3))
 (segment (start 69.85 45.212) (end 69.85 44.704) (width 1.5) (layer B.Cu) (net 3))
 (segment (start 66.802 48.26) (end 69.85 45.212) (width 1.5) (layer B.Cu) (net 3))
 (segment (start 64.008 54.356) (end 64.008 53.086) (width 1.5) (layer B.Cu) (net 3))
 (segment (start 64.008 53.086) (end 66.802 50.292) (width 1.5) (layer B.Cu) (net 3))
 (segment (start 66.802 50.292) (end 66.802 48.768) (width 1.5) (layer B.Cu) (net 3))
 (segment (start 47.244 54.102) (end 48.514 54.102) (width 1.5) (layer B.Cu) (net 3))
 (segment (start 55.626 55.118) (end 56.388 54.356) (width 1.5) (layer B.Cu) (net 3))
 (segment (start 49.53 55.118) (end 55.626 55.118) (width 1.5) (layer B.Cu) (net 3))
 (segment (start 48.514 54.102) (end 49.53 55.118) (width 1.5) (layer B.Cu) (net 3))
 (segment (start 74.93 48.514) (end 75.692 48.514) (width 1) (layer B.Cu) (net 13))
 (segment (start 100.6435 41.2075) (end 100.684 41.2075) (width 1) (layer F.Cu) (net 13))
 (segment (start 100.584 41.148) (end 100.6435 41.2075) (width 1) (layer F.Cu) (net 13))
 (via (at 100.584 41.148) (size 1.5) (drill 0.8) (layers F.Cu B.Cu) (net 13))
 (segment (start 100.584 42.418) (end 100.584 41.148) (width 1) (layer B.Cu) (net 13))
 (segment (start 99.568 43.434) (end 100.584 42.418) (width 1) (layer B.Cu) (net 13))
 (segment (start 85.598 43.434) (end 99.568 43.434) (width 1) (layer B.Cu) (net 13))
 (segment (start 84.836 44.196) (end 85.598 43.434) (width 1) (layer B.Cu) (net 13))
 (segment (start 84.836 45.72) (end 84.836 44.196) (width 1) (layer B.Cu) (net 13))
 (segment (start 83.82 46.736) (end 84.836 45.72) (width 1) (layer B.Cu) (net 13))
 (segment (start 77.47 46.736) (end 83.82 46.736) (width 1) (layer B.Cu) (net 13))
 (segment (start 75.692 48.514) (end 77.47 46.736) (width 1) (layer B.Cu) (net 13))
 (segment (start 72.39 52.832) (end 72.39 52.07) (width 1) (layer B.Cu) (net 12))
 (segment (start 102.6755 41.2075) (end 102.684 41.2075) (width 1) (layer F.Cu) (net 12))
 (segment (start 102.616 41.148) (end 102.6755 41.2075) (width 1) (layer F.Cu) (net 12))
 (via (at 102.616 41.148) (size 1.5) (drill 0.8) (layers F.Cu B.Cu) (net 12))
 (segment (start 102.616 42.418) (end 102.616 41.148) (width 1) (layer B.Cu) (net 12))
 (segment (start 104.902 44.704) (end 102.616 42.418) (width 1) (layer B.Cu) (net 12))
 (segment (start 104.902 48.006) (end 104.902 44.704) (width 1) (layer B.Cu) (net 12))
 (segment (start 103.632 49.276) (end 104.902 48.006) (width 1) (layer B.Cu) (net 12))
 (segment (start 85.09 49.276) (end 103.632 49.276) (width 1) (layer B.Cu) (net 12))
 (segment (start 84.074 48.26) (end 85.09 49.276) (width 1) (layer B.Cu) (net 12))
 (segment (start 78.232 48.26) (end 84.074 48.26) (width 1) (layer B.Cu) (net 12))
 (segment (start 75.946 50.546) (end 78.232 48.26) (width 1) (layer B.Cu) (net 12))
 (segment (start 73.914 50.546) (end 75.946 50.546) (width 1) (layer B.Cu) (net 12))
 (segment (start 72.39 52.07) (end 73.914 50.546) (width 1) (layer B.Cu) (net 12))
 (segment (start 81.28 52.832) (end 86.487 52.832) (width 1.5) (layer B.Cu) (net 1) (status 30))
 (segment (start 86.487 52.832) (end 87.122 53.467) (width 1.5) (layer B.Cu) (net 1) (status 30))
 (segment (start 107.188 32.512) (end 107.188 31.75) (width 1) (layer B.Cu) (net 15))
 (segment (start 107.188 31.75) (end 102.616 27.178) (width 1) (layer B.Cu) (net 15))
 (segment (start 102.684 24.198) (end 102.684 24.3245) (width 1) (layer F.Cu) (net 15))
 (segment (start 102.616 24.13) (end 102.684 24.198) (width 1) (layer F.Cu) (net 15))
 (via (at 102.616 24.13) (size 1.5) (drill 0.8) (layers F.Cu B.Cu) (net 15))
 (segment (start 102.616 27.178) (end 102.616 24.13) (width 1) (layer B.Cu) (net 15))
 (segment (start 70.104 53.34) (end 71.628 54.864) (width 1) (layer B.Cu) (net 15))
 (segment (start 103.378 27.94) (end 105.029 29.591) (width 1) (layer B.Cu) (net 15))
 (segment (start 105.029 29.591) (end 107.188 31.75) (width 1) (layer B.Cu) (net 15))
 (segment (start 107.188 32.512) (end 107.188 40.132) (width 1) (layer B.Cu) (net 15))
 (segment (start 107.188 40.132) (end 107.95 40.894) (width 1) (layer B.Cu) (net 15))
 (segment (start 70.104 53.34) (end 70.104 52.832) (width 1) (layer B.Cu) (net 15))
 (segment (start 108.966 41.91) (end 107.95 40.894) (width 1) (layer B.Cu) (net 15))
 (segment (start 109.728 41.91) (end 108.966 41.91) (width 1) (layer B.Cu) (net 15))
 (segment (start 109.982 42.164) (end 109.728 41.91) (width 1) (layer B.Cu) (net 15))
 (via (at 109.982 42.164) (size 1.5) (drill 0.8) (layers F.Cu B.Cu) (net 15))
 (segment (start 109.982 48.768) (end 109.982 42.164) (width 1) (layer F.Cu) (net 15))
 (segment (start 108.204 50.546) (end 109.982 48.768) (width 1) (layer F.Cu) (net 15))
 (segment (start 86.106 50.546) (end 108.204 50.546) (width 1) (layer F.Cu) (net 15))
 (segment (start 84.074 52.578) (end 86.106 50.546) (width 1) (layer F.Cu) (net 15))
 (segment (start 84.074 54.102) (end 84.074 52.578) (width 1) (layer F.Cu) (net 15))
 (segment (start 83.312 54.864) (end 84.074 54.102) (width 1) (layer F.Cu) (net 15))
 (via (at 83.312 54.864) (size 1.5) (drill 0.8) (layers F.Cu B.Cu) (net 15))
 (segment (start 71.628 54.864) (end 83.312 54.864) (width 1) (layer B.Cu) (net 15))
 (segment (start 56.388 49.276) (end 64.008 49.276) (width 1.5) (layer B.Cu) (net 6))
 (segment (start 64.008 49.276) (end 64.008 48.26) (width 1) (layer F.Cu) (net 6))
 (segment (start 87.122 26.67) (end 87.63 27.178) (width 1) (layer F.Cu) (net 6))
 (segment (start 76.708 26.67) (end 87.122 26.67) (width 1) (layer F.Cu) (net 6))
 (segment (start 73.406 29.972) (end 76.708 26.67) (width 1) (layer F.Cu) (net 6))
 (via (at 73.406 29.972) (size 1.5) (drill 0.8) (layers F.Cu B.Cu) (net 6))
 (segment (start 67.31 36.068) (end 73.406 29.972) (width 1) (layer B.Cu) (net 6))
 (segment (start 67.31 39.878) (end 67.31 36.068) (width 1) (layer B.Cu) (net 6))
 (segment (start 67.056 40.132) (end 67.31 39.878) (width 1) (layer B.Cu) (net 6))
 (via (at 67.056 40.132) (size 1.5) (drill 0.8) (layers F.Cu B.Cu) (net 6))
 (segment (start 67.056 45.212) (end 67.056 40.132) (width 1) (layer F.Cu) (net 6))
 (segment (start 64.008 48.26) (end 67.056 45.212) (width 1) (layer F.Cu) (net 6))
 (segment (start 87.63 27.178) (end 87.864002 27.178) (width 1) (layer F.Cu) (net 6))
 (segment (start 87.864002 27.178) (end 88.880002 26.162) (width 1) (layer F.Cu) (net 6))
 (segment (start 88.880002 26.162) (end 91.694 26.162) (width 1) (layer F.Cu) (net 6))
 (segment (start 91.694 26.162) (end 92.964 27.432) (width 1) (layer F.Cu) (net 6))
 (segment (start 92.964 27.432) (end 105.156 27.432) (width 1) (layer F.Cu) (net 6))
 (segment (start 105.156 27.432) (end 106.684 25.904) (width 1) (layer F.Cu) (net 6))
 (segment (start 87.864002 27.178) (end 88.880002 26.162) (width 1) (layer F.Cu) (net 6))
 (segment (start 106.684 25.904) (end 106.684 24.3245) (width 1) (layer F.Cu) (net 6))
 (segment (start 39.624 49.022) (end 47.244 49.022) (width 1.5) (layer B.Cu) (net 7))
 (segment (start 54.102 33.274) (end 48.26 33.274) (width 1) (layer F.Cu) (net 7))
 (segment (start 39.624 41.91) (end 39.624 49.022) (width 1) (layer F.Cu) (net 7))
 (segment (start 48.26 33.274) (end 39.624 41.91) (width 1) (layer F.Cu) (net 7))
 (segment (start 98.806 37.846) (end 98.806 36.83) (width 1) (layer B.Cu) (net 7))
 (segment (start 77.47 33.274) (end 54.102 33.274) (width 1) (layer F.Cu) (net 7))
 (segment (start 54.102 33.274) (end 53.848 33.274) (width 1) (layer F.Cu) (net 7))
 (via (at 77.47 33.274) (size 1.5) (drill 0.8) (layers F.Cu B.Cu) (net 7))
 (segment (start 95.25 33.274) (end 77.47 33.274) (width 1) (layer B.Cu) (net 7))
 (segment (start 98.806 36.83) (end 95.25 33.274) (width 1) (layer B.Cu) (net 7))
 (via (at 98.684 41.2075) (size 1.5) (drill 0.8) (layers F.Cu B.Cu) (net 7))
 (segment (start 98.806 37.338) (end 98.806 37.846) (width 1) (layer B.Cu) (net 7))
 (segment (start 98.806 37.846) (end 98.806 41.0855) (width 1) (layer B.Cu) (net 7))
 (segment (start 98.806 41.0855) (end 98.684 41.2075) (width 1) (layer B.Cu) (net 7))
 (segment (start 47.244 49.022) (end 49.276 49.022) (width 1.5) (layer B.Cu) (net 7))
 (segment (start 49.276 49.022) (end 50.546 50.292) (width 1.5) (layer B.Cu) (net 7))
 (segment (start 57.658 34.798) (end 57.15 34.798) (width 1) (layer F.Cu) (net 10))
 (segment (start 53.34 38.608) (end 53.34 46.99) (width 1) (layer F.Cu) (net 10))
 (segment (start 57.15 34.798) (end 53.34 38.608) (width 1) (layer F.Cu) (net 10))
 (segment (start 96.774 38.1) (end 96.774 37.846) (width 1) (layer B.Cu) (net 10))
 (segment (start 79.756 34.798) (end 57.658 34.798) (width 1) (layer F.Cu) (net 10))
 (via (at 79.756 34.798) (size 1.5) (drill 0.8) (layers F.Cu B.Cu) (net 10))
 (segment (start 93.726 34.798) (end 79.756 34.798) (width 1) (layer B.Cu) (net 10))
 (segment (start 96.774 37.846) (end 93.726 34.798) (width 1) (layer B.Cu) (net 10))
 (via (at 96.7105 41.2115) (size 1.5) (drill 0.8) (layers F.Cu B.Cu) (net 10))
 (segment (start 96.774 38.1) (end 96.774 41.148) (width 1) (layer B.Cu) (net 10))
 (segment (start 96.774 41.148) (end 96.7105 41.2115) (width 1) (layer B.Cu) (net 10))
 (segment (start 69.342 48.768) (end 72.136 48.768) (width 1) (layer B.Cu) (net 14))
 (segment (start 72.136 48.768) (end 72.39 48.514) (width 1) (layer B.Cu) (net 14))
 (segment (start 85.852 41.148) (end 85.852 42.418) (width 1) (layer F.Cu) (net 11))
 (segment (start 94.684 42.984) (end 94.684 41.2075) (width 1) (layer F.Cu) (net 11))
 (segment (start 94.234 43.434) (end 94.684 42.984) (width 1) (layer F.Cu) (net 11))
 (segment (start 86.868 43.434) (end 94.234 43.434) (width 1) (layer F.Cu) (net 11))
 (segment (start 85.852 42.418) (end 86.868 43.434) (width 1) (layer F.Cu) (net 11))
 (segment (start 74.93 52.832) (end 78.74 52.832) (width 1) (layer B.Cu) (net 2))
 (segment (start 78.74 52.832) (end 81.28 50.292) (width 1) (layer B.Cu) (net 2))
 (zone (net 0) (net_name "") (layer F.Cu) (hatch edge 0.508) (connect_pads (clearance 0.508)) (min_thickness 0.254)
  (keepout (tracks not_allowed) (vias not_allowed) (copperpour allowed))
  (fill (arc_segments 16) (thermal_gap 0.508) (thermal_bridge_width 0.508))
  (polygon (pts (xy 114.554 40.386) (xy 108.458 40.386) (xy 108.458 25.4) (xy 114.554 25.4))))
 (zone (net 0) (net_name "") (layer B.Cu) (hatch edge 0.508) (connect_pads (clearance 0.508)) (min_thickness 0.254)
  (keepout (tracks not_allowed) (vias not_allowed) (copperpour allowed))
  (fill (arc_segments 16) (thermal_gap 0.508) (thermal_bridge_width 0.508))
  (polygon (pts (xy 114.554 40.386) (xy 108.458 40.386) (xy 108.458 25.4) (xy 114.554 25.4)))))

